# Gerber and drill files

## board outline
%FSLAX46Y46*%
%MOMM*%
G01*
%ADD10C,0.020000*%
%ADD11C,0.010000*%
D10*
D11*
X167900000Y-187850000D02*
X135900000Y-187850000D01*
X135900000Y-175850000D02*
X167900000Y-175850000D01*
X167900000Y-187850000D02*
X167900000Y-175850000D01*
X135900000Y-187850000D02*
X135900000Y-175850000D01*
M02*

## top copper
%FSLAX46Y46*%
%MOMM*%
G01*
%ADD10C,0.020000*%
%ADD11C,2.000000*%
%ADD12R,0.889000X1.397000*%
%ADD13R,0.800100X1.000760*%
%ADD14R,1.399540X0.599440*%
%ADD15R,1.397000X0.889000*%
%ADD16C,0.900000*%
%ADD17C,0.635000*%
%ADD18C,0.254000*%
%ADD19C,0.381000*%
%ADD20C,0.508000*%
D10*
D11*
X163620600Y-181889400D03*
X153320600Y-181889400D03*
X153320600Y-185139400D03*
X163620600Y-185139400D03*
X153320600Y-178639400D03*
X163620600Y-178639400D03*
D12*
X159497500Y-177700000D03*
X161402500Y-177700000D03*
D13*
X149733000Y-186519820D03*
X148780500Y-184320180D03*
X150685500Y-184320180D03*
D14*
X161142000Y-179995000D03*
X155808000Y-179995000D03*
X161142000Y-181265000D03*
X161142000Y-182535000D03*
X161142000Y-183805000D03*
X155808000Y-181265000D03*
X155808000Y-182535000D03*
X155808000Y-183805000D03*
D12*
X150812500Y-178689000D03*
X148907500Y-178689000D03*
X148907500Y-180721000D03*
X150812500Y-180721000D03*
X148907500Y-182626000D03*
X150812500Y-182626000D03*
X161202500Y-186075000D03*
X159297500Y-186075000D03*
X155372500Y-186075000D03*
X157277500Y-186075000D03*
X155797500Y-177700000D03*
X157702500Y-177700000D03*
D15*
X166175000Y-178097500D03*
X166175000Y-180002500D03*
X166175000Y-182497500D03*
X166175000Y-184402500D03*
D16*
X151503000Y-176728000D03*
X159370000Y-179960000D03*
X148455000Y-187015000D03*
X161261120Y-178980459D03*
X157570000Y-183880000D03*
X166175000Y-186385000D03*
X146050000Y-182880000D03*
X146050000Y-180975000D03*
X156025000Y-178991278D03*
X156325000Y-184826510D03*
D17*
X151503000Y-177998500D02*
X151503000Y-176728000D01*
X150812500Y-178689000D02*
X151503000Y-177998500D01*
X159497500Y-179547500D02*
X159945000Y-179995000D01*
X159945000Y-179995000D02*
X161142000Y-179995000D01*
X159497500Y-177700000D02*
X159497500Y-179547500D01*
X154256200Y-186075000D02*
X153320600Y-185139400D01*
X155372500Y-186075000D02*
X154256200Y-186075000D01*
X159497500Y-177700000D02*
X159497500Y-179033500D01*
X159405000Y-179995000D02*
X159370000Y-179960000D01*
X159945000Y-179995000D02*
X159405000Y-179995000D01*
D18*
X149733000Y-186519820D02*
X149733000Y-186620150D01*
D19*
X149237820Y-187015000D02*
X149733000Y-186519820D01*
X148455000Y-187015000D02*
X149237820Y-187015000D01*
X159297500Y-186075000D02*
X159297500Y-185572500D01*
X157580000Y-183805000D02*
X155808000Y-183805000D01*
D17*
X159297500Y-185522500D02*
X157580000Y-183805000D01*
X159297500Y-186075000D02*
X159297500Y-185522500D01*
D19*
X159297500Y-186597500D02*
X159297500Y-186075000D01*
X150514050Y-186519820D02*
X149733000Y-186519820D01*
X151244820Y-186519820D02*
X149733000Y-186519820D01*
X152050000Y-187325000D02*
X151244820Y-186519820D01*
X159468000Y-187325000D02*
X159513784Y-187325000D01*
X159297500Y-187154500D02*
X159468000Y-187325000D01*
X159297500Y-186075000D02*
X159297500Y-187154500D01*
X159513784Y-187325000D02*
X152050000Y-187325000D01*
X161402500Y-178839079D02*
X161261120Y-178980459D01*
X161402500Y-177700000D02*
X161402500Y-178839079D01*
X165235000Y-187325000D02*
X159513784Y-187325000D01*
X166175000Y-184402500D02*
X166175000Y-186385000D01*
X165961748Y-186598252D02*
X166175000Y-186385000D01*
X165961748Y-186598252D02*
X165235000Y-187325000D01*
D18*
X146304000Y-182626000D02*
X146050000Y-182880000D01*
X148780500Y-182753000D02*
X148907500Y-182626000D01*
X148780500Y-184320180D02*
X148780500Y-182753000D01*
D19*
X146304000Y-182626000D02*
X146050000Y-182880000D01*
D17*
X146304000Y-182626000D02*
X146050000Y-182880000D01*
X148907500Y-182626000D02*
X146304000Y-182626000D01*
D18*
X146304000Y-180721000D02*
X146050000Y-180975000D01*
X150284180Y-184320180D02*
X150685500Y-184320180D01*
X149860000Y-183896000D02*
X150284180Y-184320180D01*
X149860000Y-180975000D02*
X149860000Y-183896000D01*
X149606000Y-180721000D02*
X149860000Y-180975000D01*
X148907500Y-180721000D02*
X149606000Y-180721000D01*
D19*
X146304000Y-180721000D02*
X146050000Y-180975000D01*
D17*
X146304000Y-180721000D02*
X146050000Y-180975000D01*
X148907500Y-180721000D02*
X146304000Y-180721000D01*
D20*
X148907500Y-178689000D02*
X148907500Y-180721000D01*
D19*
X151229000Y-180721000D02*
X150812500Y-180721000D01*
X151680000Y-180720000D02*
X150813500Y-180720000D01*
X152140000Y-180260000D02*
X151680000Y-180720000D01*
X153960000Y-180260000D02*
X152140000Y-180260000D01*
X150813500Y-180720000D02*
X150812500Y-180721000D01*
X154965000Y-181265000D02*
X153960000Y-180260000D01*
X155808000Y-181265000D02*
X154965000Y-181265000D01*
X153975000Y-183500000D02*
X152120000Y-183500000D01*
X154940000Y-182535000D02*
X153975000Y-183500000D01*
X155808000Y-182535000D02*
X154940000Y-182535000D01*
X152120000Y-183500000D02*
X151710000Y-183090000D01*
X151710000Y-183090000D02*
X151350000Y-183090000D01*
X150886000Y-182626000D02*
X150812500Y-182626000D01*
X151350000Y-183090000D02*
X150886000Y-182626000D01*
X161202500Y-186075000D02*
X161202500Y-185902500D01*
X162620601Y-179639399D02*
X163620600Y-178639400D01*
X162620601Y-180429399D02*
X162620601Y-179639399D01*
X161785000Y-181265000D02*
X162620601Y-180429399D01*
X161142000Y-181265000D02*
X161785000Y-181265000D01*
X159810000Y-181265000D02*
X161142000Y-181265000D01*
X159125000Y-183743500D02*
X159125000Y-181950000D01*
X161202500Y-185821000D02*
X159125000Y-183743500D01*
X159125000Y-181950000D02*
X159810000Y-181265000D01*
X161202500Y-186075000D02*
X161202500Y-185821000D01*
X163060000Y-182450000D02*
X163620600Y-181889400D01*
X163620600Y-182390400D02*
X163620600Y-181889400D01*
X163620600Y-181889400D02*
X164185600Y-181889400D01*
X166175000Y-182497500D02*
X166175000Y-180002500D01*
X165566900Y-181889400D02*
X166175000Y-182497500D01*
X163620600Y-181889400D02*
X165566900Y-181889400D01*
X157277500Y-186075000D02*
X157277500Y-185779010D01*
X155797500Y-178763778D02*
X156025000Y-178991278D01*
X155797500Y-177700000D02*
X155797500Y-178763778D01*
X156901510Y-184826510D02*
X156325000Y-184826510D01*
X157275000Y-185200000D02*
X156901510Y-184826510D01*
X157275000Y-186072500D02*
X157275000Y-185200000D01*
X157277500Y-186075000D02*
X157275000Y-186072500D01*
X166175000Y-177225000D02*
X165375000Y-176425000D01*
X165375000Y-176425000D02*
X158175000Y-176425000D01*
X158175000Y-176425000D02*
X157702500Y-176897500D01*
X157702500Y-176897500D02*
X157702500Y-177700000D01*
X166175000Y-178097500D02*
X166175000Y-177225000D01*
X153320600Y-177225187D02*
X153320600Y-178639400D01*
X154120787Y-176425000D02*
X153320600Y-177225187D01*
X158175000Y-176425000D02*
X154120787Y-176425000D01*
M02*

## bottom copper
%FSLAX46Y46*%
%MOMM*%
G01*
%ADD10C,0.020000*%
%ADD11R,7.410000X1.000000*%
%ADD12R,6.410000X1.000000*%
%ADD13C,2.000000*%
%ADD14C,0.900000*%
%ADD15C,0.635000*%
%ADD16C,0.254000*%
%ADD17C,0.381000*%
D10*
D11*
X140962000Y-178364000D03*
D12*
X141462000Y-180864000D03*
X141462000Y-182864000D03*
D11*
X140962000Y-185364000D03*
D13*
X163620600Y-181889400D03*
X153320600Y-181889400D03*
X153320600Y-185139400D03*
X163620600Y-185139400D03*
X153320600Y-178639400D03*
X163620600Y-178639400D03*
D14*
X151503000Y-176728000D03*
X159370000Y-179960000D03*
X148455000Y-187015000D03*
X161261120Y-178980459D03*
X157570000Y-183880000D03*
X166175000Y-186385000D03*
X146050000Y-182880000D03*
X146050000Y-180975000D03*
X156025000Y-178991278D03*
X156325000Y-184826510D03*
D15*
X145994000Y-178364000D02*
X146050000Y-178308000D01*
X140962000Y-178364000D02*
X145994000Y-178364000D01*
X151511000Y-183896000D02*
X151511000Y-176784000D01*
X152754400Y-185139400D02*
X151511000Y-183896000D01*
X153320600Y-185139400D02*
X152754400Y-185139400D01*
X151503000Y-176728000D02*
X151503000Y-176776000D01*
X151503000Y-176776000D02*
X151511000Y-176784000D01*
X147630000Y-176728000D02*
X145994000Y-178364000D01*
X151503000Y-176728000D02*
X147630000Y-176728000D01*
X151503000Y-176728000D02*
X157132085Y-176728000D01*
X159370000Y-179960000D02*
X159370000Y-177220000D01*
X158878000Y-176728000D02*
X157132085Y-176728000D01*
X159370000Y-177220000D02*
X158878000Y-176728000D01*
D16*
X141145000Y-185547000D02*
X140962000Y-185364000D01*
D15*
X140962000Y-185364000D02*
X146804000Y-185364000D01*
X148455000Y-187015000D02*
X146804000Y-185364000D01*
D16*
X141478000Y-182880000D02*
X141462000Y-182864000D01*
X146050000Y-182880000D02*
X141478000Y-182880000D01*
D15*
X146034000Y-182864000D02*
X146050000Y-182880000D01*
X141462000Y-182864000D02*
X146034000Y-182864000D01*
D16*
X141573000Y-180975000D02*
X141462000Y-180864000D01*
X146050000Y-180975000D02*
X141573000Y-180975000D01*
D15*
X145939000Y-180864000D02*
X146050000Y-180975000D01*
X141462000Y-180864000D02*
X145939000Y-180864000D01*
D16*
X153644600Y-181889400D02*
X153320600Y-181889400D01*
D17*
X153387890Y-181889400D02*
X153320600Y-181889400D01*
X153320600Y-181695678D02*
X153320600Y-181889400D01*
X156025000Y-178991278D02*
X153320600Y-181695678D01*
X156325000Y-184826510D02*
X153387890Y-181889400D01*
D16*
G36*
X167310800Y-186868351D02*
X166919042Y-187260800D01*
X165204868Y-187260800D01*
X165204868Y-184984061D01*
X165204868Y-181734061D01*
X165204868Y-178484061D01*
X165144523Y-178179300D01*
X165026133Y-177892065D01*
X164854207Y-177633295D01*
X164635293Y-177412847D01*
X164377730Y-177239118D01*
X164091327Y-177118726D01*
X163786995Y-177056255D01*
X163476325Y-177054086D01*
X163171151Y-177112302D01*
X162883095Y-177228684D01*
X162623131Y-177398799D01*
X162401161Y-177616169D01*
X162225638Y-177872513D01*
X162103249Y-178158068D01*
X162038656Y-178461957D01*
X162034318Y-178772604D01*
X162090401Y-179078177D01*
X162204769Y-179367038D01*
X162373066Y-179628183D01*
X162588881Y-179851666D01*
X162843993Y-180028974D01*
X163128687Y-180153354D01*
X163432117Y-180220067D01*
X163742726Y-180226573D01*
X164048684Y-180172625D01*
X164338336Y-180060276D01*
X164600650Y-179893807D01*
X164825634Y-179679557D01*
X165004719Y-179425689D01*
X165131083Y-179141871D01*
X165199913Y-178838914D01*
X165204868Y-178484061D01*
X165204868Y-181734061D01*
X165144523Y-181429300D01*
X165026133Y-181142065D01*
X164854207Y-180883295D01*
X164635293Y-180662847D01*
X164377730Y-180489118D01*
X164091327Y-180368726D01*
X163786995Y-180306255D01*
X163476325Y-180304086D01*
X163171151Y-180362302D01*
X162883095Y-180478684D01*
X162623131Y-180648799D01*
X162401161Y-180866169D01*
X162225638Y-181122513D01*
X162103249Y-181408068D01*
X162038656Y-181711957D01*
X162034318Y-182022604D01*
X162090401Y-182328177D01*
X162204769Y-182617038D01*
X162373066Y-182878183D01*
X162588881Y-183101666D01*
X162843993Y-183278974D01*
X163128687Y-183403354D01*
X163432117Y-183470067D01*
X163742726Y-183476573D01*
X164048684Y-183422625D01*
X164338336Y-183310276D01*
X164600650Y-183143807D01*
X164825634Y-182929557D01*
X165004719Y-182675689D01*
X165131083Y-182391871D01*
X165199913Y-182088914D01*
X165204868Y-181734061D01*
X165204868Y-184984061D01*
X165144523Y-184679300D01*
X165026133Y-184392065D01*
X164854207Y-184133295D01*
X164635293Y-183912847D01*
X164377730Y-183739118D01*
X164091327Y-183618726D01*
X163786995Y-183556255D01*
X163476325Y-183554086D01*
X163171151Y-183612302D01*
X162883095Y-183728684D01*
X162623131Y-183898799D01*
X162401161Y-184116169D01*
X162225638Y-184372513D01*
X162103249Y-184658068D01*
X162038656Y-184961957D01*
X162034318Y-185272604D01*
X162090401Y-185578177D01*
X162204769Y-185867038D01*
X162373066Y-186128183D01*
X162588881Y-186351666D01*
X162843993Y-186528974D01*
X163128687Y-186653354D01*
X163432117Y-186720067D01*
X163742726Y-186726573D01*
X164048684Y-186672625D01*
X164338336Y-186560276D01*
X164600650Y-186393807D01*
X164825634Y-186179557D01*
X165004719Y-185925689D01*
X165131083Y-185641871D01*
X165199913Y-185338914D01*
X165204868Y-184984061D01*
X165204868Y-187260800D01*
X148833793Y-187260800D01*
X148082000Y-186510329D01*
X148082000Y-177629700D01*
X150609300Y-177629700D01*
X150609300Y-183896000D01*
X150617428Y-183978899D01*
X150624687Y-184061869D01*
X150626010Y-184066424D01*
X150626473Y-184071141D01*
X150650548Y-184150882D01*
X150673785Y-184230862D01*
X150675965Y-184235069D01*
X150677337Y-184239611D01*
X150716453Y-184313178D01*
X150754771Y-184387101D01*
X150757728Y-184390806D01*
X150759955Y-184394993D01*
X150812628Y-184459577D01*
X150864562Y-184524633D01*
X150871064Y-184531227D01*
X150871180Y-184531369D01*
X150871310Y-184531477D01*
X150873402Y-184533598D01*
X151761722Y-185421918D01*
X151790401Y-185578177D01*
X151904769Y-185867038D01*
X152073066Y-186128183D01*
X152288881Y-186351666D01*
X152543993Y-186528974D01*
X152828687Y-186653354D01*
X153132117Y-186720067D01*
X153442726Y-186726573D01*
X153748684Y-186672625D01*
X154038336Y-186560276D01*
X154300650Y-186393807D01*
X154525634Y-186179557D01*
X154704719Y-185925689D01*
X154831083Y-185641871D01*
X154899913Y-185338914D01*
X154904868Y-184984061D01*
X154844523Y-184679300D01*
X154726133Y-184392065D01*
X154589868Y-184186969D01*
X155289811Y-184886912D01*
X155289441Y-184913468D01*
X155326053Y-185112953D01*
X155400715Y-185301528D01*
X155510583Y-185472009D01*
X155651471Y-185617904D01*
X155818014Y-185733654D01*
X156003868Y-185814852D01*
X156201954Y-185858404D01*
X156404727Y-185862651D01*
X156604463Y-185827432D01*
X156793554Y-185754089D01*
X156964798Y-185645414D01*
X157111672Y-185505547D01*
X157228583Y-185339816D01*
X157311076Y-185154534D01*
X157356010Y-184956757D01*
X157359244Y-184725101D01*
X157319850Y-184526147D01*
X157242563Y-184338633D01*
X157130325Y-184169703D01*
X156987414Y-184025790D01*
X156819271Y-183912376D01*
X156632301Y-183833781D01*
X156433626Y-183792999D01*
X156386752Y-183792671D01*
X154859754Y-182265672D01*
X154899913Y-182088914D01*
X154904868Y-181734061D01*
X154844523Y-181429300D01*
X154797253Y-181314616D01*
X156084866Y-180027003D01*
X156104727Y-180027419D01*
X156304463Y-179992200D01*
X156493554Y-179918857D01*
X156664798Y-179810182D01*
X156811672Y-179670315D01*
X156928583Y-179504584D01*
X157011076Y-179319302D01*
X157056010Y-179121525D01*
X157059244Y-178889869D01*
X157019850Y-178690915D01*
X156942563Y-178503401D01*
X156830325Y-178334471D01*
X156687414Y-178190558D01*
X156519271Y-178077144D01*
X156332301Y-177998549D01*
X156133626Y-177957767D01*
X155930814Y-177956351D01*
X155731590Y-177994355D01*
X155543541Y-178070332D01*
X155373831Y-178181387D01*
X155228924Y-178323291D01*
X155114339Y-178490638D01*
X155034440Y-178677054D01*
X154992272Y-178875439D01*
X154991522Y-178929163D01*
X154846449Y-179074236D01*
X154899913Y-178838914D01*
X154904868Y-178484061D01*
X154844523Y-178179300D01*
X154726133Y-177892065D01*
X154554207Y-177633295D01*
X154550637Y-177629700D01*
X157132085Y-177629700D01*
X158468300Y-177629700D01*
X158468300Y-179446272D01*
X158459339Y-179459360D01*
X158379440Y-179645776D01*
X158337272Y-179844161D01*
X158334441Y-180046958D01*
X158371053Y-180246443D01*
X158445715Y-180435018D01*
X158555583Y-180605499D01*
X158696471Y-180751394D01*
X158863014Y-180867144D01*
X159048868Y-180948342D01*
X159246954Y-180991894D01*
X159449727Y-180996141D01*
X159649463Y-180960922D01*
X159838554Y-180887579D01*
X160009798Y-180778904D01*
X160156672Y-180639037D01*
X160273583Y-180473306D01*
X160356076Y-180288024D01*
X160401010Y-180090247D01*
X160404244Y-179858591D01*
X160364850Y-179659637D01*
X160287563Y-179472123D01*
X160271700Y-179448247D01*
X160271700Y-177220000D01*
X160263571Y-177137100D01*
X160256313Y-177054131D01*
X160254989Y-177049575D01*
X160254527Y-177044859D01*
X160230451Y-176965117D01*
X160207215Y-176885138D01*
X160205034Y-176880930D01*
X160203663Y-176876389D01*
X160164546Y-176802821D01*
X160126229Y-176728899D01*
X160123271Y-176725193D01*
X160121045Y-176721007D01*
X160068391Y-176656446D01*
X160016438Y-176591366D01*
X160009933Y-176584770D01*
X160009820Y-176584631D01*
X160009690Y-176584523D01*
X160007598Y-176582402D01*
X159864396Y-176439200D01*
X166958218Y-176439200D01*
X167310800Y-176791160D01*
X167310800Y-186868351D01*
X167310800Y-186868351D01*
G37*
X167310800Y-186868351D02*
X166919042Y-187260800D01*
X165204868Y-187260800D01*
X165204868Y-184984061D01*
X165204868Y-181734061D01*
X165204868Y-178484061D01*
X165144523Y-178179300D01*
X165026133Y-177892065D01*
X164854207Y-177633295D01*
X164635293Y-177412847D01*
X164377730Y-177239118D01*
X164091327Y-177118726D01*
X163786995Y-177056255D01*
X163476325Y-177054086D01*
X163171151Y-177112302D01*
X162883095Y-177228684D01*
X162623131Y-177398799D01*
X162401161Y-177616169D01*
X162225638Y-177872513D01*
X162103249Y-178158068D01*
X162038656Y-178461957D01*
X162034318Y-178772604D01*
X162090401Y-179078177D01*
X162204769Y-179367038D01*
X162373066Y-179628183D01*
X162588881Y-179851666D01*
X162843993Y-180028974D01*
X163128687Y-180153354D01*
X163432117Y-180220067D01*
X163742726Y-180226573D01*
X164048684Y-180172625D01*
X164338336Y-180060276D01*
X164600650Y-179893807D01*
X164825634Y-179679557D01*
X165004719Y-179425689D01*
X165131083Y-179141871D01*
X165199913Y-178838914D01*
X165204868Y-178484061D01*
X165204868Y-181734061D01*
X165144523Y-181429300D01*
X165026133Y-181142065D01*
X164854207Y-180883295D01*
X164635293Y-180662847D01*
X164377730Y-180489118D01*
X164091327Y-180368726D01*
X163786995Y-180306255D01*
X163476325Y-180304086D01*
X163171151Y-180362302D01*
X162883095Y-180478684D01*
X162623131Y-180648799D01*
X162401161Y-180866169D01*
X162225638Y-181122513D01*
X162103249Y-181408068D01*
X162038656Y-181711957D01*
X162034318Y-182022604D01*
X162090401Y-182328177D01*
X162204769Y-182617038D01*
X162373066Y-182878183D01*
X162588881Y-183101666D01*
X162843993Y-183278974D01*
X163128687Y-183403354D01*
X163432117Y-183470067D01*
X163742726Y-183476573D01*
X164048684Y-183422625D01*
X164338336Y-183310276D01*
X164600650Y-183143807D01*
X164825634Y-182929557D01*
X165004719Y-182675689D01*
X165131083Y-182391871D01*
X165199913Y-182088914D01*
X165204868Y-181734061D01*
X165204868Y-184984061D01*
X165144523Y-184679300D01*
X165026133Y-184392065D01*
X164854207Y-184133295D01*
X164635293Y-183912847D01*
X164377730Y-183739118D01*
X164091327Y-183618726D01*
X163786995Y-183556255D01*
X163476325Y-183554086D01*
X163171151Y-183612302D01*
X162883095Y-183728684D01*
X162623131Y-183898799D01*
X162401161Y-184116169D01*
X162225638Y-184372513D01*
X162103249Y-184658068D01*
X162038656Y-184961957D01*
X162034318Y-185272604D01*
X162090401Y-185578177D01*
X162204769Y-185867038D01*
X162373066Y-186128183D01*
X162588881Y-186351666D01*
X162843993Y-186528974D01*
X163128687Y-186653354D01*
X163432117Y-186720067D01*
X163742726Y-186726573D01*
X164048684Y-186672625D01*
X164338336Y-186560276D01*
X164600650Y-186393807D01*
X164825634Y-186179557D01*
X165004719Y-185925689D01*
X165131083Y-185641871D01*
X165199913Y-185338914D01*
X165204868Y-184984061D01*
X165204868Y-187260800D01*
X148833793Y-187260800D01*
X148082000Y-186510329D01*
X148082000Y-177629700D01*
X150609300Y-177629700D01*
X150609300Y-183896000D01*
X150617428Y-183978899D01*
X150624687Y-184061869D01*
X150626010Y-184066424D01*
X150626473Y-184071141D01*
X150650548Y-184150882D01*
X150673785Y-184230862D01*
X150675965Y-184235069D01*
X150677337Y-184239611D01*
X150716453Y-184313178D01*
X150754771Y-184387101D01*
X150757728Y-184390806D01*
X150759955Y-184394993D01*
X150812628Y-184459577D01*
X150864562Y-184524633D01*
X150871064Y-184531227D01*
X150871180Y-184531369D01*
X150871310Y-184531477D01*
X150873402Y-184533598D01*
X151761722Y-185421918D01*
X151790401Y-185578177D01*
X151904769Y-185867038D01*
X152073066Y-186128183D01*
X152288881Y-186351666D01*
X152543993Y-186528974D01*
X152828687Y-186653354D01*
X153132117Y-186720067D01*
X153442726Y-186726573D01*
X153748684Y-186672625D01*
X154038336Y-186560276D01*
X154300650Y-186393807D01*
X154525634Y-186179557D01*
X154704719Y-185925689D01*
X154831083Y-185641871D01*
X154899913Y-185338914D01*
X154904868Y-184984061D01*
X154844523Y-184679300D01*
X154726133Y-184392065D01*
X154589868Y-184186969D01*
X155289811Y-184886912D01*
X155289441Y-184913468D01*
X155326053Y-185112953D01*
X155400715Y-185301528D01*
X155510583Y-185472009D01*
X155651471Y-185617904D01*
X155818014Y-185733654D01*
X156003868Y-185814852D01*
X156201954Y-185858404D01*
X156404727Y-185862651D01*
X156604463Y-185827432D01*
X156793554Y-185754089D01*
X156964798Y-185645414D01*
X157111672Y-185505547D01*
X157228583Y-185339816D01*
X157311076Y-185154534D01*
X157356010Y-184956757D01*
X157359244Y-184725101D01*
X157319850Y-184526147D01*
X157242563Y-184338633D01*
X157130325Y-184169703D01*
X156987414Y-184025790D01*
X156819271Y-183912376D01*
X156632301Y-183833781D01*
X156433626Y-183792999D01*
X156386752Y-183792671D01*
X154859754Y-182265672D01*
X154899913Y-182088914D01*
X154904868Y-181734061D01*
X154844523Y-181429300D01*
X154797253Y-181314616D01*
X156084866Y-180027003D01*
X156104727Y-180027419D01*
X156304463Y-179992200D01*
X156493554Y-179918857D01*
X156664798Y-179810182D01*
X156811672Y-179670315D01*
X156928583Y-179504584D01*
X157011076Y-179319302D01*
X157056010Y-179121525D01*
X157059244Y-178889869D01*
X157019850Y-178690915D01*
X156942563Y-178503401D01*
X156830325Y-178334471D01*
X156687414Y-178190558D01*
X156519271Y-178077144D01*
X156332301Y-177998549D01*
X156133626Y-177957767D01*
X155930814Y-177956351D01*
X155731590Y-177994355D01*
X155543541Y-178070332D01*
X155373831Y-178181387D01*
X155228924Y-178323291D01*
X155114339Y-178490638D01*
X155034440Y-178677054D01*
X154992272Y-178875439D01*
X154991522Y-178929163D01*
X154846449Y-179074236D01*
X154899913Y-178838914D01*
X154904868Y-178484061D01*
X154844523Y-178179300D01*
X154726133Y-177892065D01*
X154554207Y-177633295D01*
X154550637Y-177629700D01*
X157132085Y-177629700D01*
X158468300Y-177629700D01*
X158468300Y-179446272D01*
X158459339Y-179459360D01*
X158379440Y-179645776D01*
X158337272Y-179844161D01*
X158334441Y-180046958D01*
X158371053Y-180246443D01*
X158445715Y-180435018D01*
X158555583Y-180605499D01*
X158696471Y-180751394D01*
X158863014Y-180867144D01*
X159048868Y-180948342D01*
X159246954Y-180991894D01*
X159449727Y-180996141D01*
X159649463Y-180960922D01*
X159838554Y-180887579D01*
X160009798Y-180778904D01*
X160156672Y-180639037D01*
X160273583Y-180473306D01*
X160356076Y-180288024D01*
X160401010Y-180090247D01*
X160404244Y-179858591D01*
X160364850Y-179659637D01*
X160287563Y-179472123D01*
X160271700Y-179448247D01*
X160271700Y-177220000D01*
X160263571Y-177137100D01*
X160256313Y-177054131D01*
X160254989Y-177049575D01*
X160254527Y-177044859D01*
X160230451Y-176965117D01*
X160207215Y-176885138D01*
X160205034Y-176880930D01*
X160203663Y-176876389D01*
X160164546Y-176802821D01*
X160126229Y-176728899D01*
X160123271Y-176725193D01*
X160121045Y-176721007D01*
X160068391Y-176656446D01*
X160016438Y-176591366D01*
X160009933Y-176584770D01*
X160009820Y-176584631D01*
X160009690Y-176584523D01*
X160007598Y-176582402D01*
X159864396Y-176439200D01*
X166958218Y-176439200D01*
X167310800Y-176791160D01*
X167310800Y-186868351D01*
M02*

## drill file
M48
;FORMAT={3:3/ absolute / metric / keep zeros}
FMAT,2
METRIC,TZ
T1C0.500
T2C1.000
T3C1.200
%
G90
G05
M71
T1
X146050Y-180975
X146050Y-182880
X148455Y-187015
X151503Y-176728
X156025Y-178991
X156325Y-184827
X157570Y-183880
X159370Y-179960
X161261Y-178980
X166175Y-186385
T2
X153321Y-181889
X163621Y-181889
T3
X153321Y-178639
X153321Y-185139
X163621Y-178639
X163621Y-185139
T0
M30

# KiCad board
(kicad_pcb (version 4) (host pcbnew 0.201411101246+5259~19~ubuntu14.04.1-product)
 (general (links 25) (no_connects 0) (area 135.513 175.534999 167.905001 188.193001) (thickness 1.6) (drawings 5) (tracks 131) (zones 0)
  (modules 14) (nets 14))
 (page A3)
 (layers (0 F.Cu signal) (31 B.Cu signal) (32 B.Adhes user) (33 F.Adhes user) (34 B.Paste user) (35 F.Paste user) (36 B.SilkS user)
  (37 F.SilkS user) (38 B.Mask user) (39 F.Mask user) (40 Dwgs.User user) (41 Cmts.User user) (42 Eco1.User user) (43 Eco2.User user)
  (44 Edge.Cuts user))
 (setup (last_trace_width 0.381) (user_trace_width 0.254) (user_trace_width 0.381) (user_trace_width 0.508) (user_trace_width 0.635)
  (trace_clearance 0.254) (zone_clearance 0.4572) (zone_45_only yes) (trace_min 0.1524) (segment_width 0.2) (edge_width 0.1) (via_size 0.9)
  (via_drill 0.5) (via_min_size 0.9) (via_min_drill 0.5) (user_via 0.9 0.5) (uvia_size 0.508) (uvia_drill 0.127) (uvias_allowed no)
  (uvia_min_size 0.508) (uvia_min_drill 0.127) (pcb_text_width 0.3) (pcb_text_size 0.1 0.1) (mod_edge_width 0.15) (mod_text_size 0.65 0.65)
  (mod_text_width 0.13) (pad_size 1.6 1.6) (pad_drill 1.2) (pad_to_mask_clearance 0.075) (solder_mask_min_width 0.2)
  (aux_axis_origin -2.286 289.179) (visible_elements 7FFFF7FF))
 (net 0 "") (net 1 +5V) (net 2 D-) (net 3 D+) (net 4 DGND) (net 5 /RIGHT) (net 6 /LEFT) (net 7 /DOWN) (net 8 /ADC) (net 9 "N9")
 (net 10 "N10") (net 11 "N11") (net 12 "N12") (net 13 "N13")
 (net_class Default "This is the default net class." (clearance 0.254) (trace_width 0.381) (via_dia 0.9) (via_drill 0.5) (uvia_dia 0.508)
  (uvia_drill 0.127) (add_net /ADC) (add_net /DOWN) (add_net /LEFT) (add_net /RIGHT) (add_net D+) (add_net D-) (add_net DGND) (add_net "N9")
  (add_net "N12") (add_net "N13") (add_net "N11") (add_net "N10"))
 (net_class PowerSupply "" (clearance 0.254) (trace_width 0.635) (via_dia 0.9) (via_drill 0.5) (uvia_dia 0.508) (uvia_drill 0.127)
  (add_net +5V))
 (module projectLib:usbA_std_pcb (layer B.Cu) (at 136.017 181.864)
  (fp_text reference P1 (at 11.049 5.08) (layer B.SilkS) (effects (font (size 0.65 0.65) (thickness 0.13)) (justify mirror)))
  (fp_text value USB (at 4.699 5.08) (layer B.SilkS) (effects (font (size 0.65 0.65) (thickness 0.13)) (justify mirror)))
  (pad 1 smd rect (at 4.945 -3.5) (size 7.41 1) (layers B.Cu B.Mask) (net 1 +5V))
  (pad 2 smd rect (at 5.445 -1) (size 6.41 1) (layers B.Cu B.Mask) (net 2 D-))
  (pad 3 smd rect (at 5.445 1) (size 6.41 1) (layers B.Cu B.Mask) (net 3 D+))
  (pad 4 smd rect (at 4.945 3.5) (size 7.41 1) (layers B.Cu B.Mask) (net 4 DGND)))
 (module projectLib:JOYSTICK (layer B.Cu) (at 158.4706 181.8894)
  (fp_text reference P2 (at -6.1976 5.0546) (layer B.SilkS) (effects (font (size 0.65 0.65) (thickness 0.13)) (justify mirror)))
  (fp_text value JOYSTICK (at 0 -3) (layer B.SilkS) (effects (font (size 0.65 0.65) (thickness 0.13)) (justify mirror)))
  (pad 5 thru_hole circle (at 5.15 0) (size 2 2) (drill 1) (layers *.Cu *.Mask B.SilkS) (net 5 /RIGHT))
  (pad 2 thru_hole circle (at -5.15 0) (size 2 2) (drill 1) (layers *.Cu *.Mask B.SilkS) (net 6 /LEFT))
  (pad 1 thru_hole circle (at -5.15 3.25) (size 2 2) (drill 1.2) (layers *.Cu *.Mask B.SilkS) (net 1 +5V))
  (pad 6 thru_hole circle (at 5.15 3.25) (size 2 2) (drill 1.2) (layers *.Cu *.Mask B.SilkS))
  (pad 3 thru_hole circle (at -5.15 -3.25) (size 2 2) (drill 1.2) (layers *.Cu *.Mask B.SilkS) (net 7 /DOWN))
  (pad 4 thru_hole circle (at 5.15 -3.25) (size 2 2) (drill 1.2) (layers *.Cu *.Mask B.SilkS) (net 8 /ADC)))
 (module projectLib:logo (layer F.Cu) (at 140.7 181.66 90)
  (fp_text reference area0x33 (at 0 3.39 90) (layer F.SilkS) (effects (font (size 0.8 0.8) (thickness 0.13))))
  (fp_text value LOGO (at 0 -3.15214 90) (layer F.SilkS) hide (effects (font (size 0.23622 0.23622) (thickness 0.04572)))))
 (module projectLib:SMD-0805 (layer F.Cu) (at 160.45 177.7)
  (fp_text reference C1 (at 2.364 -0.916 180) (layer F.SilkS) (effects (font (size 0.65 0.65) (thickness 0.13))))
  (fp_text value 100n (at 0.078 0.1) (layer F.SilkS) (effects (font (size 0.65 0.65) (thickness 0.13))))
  (pad 1 smd rect (at -0.9525 0) (size 0.889 1.397) (layers F.Cu F.Paste F.Mask) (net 1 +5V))
  (pad 2 smd rect (at 0.9525 0) (size 0.889 1.397) (layers F.Cu F.Paste F.Mask) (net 4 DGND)))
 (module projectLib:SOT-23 (layer F.Cu) (at 149.733 185.42 180)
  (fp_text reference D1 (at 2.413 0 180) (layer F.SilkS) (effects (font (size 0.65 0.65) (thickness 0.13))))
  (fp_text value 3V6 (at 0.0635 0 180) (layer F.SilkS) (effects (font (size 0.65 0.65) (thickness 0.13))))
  (pad 3 smd rect (at 0 -1.09982 180) (size 0.8001 1.00076) (layers F.Cu F.Paste F.Mask) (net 4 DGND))
  (pad 2 smd rect (at 0.9525 1.09982 180) (size 0.8001 1.00076) (layers F.Cu F.Paste F.Mask) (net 3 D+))
  (pad 1 smd rect (at -0.9525 1.09982 180) (size 0.8001 1.00076) (layers F.Cu F.Paste F.Mask) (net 2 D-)))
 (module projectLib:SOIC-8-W (layer F.Cu) (at 158.475 181.9 270)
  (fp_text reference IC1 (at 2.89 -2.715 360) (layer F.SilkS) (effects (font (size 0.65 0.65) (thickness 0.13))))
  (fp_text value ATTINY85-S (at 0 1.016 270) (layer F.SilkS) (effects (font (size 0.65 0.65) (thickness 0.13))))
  (pad 8 smd rect (at -1.905 -2.667 270) (size 0.59944 1.39954) (layers F.Cu F.Paste F.Mask) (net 1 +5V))
  (pad 1 smd rect (at -1.905 2.667 270) (size 0.59944 1.39954) (layers F.Cu F.Paste F.Mask) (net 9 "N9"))
  (pad 7 smd rect (at -0.635 -2.667 270) (size 0.59944 1.39954) (layers F.Cu F.Paste F.Mask) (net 8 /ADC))
  (pad 6 smd rect (at 0.635 -2.667 270) (size 0.59944 1.39954) (layers F.Cu F.Paste F.Mask) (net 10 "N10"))
  (pad 5 smd rect (at 1.905 -2.667 270) (size 0.59944 1.39954) (layers F.Cu F.Paste F.Mask) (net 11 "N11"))
  (pad 2 smd rect (at -0.635 2.667 270) (size 0.59944 1.39954) (layers F.Cu F.Paste F.Mask) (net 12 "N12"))
  (pad 3 smd rect (at 0.635 2.667 270) (size 0.59944 1.39954) (layers F.Cu F.Paste F.Mask) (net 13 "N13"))
  (pad 4 smd rect (at 1.905 2.667 270) (size 0.59944 1.39954) (layers F.Cu F.Paste F.Mask) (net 4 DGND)))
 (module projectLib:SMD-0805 (layer F.Cu) (at 149.86 178.689 180)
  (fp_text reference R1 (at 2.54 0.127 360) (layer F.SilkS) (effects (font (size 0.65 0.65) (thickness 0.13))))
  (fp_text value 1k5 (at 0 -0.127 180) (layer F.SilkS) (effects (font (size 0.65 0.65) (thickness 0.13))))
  (pad 1 smd rect (at -0.9525 0 180) (size 0.889 1.397) (layers F.Cu F.Paste F.Mask) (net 1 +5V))
  (pad 2 smd rect (at 0.9525 0 180) (size 0.889 1.397) (layers F.Cu F.Paste F.Mask) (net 2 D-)))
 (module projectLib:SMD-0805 (layer F.Cu) (at 149.86 180.721)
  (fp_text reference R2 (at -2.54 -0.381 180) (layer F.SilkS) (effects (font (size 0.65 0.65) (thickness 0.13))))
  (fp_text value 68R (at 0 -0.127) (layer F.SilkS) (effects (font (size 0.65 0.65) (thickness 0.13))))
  (pad 1 smd rect (at -0.9525 0) (size 0.889 1.397) (layers F.Cu F.Paste F.Mask) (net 2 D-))
  (pad 2 smd rect (at 0.9525 0) (size 0.889 1.397) (layers F.Cu F.Paste F.Mask) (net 12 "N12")))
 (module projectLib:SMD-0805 (layer F.Cu) (at 149.86 182.626)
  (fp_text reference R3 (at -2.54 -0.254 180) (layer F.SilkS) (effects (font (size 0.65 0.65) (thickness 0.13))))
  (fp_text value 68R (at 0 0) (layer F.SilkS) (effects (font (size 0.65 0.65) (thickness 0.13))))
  (pad 1 smd rect (at -0.9525 0) (size 0.889 1.397) (layers F.Cu F.Paste F.Mask) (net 3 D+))
  (pad 2 smd rect (at 0.9525 0) (size 0.889 1.397) (layers F.Cu F.Paste F.Mask) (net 13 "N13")))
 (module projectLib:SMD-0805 (layer F.Cu) (at 160.25 186.075 180)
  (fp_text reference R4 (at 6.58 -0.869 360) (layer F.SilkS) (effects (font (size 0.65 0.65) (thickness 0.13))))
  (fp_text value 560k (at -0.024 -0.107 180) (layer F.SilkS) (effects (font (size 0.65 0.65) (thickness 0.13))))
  (pad 1 smd rect (at -0.9525 0 180) (size 0.889 1.397) (layers F.Cu F.Paste F.Mask) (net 8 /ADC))
  (pad 2 smd rect (at 0.9525 0 180) (size 0.889 1.397) (layers F.Cu F.Paste F.Mask) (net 4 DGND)))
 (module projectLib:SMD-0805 (layer F.Cu) (at 156.325 186.075)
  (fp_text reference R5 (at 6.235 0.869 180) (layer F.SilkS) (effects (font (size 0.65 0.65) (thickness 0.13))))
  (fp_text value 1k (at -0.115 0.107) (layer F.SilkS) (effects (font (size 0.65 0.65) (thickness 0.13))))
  (pad 1 smd rect (at -0.9525 0) (size 0.889 1.397) (layers F.Cu F.Paste F.Mask) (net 1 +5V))
  (pad 2 smd rect (at 0.9525 0) (size 0.889 1.397) (layers F.Cu F.Paste F.Mask) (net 6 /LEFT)))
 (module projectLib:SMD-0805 (layer F.Cu) (at 156.75 177.7)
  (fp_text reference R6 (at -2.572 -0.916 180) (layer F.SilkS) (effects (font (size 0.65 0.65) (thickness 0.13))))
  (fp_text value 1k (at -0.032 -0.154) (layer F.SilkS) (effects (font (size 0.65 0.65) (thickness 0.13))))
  (pad 1 smd rect (at -0.9525 0) (size 0.889 1.397) (layers F.Cu F.Paste F.Mask) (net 6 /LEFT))
  (pad 2 smd rect (at 0.9525 0) (size 0.889 1.397) (layers F.Cu F.Paste F.Mask) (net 7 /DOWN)))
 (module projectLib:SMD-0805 (layer F.Cu) (at 166.175 179.05 270)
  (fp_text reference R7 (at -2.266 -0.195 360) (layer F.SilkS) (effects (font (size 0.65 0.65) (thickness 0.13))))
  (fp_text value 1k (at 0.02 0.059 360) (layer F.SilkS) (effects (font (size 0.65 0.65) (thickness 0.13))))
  (pad 1 smd rect (at -0.9525 0 270) (size 0.889 1.397) (layers F.Cu F.Paste F.Mask) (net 7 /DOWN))
  (pad 2 smd rect (at 0.9525 0 270) (size 0.889 1.397) (layers F.Cu F.Paste F.Mask) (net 5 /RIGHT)))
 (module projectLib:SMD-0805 (layer F.Cu) (at 166.175 183.45 270)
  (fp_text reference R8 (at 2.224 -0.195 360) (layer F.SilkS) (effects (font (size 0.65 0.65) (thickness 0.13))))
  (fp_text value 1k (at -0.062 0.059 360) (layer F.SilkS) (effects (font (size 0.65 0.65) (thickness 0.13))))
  (pad 1 smd rect (at -0.9525 0 270) (size 0.889 1.397) (layers F.Cu F.Paste F.Mask) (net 5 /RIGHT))
  (pad 2 smd rect (at 0.9525 0 270) (size 0.889 1.397) (layers F.Cu F.Paste F.Mask) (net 4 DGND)))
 (gr_line (start 167.9 187.85) (end 135.9 187.85) (angle 90) (layer Edge.Cuts) (width 0.01))
 (gr_line (start 135.9 175.85) (end 167.9 175.85) (angle 90) (layer Edge.Cuts) (width 0.01))
 (gr_line (start 167.9 187.85) (end 167.9 175.85) (angle 90) (layer Edge.Cuts) (width 0.01))
 (gr_line (start 135.9 187.85) (end 135.9 175.85) (angle 90) (layer Edge.Cuts) (width 0.01))
 (segment (start 159.37 177.22) (end 158.878 176.728) (width 0.635) (layer B.Cu) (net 1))
 (segment (start 158.878 176.728) (end 157.132085 176.728) (width 0.635) (layer B.Cu) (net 1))
 (segment (start 159.37 179.96) (end 159.37 177.22) (width 0.635) (layer B.Cu) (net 1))
 (segment (start 159.945 179.995) (end 159.405 179.995) (width 0.635) (layer F.Cu) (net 1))
 (segment (start 159.405 179.995) (end 159.37 179.96) (width 0.635) (layer F.Cu) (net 1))
 (via (at 159.37 179.96) (size 0.9) (drill 0.5) (layers F.Cu B.Cu) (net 1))
 (segment (start 151.503 176.728) (end 157.132085 176.728) (width 0.635) (layer B.Cu) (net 1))
 (segment (start 159.4975 177.7) (end 159.4975 179.0335) (width 0.635) (layer F.Cu) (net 1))
 (segment (start 155.3725 186.075) (end 154.2562 186.075) (width 0.635) (layer F.Cu) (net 1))
 (segment (start 154.2562 186.075) (end 153.3206 185.1394) (width 0.635) (layer F.Cu) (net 1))
 (segment (start 159.4975 177.7) (end 159.4975 179.5475) (width 0.635) (layer F.Cu) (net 1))
 (segment (start 159.945 179.995) (end 161.142 179.995) (width 0.635) (layer F.Cu) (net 1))
 (segment (start 159.4975 179.5475) (end 159.945 179.995) (width 0.635) (layer F.Cu) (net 1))
 (segment (start 151.503 176.728) (end 147.63 176.728) (width 0.635) (layer B.Cu) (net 1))
 (segment (start 147.63 176.728) (end 145.994 178.364) (width 0.635) (layer B.Cu) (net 1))
 (segment (start 150.8125 178.689) (end 151.503 177.9985) (width 0.635) (layer F.Cu) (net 1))
 (segment (start 151.503 176.776) (end 151.511 176.784) (width 0.635) (layer B.Cu) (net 1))
 (segment (start 151.503 176.728) (end 151.503 176.776) (width 0.635) (layer B.Cu) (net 1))
 (via (at 151.503 176.728) (size 0.9) (drill 0.5) (layers F.Cu B.Cu) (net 1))
 (segment (start 151.503 177.9985) (end 151.503 176.728) (width 0.635) (layer F.Cu) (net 1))
 (segment (start 153.3206 185.1394) (end 152.7544 185.1394) (width 0.635) (layer B.Cu) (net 1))
 (segment (start 152.7544 185.1394) (end 151.511 183.896) (width 0.635) (layer B.Cu) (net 1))
 (segment (start 151.511 183.896) (end 151.511 176.784) (width 0.635) (layer B.Cu) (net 1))
 (segment (start 140.962 178.364) (end 145.994 178.364) (width 0.635) (layer B.Cu) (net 1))
 (segment (start 145.994 178.364) (end 146.05 178.308) (width 0.635) (layer B.Cu) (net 1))
 (segment (start 165.961748 186.598252) (end 165.235 187.325) (width 0.381) (layer F.Cu) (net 4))
 (segment (start 165.961748 186.598252) (end 166.175 186.385) (width 0.381) (layer F.Cu) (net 4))
 (via (at 166.175 186.385) (size 0.9) (drill 0.5) (layers F.Cu B.Cu) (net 4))
 (segment (start 166.175 184.4025) (end 166.175 186.385) (width 0.381) (layer F.Cu) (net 4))
 (segment (start 165.235 187.325) (end 159.513784 187.325) (width 0.381) (layer F.Cu) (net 4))
 (via (at 157.57 183.88) (size 0.9) (drill 0.5) (layers F.Cu B.Cu) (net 4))
 (segment (start 161.4025 177.7) (end 161.4025 178.839079) (width 0.381) (layer F.Cu) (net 4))
 (segment (start 161.4025 178.839079) (end 161.26112 178.980459) (width 0.381) (layer F.Cu) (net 4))
 (via (at 161.26112 178.980459) (size 0.9) (drill 0.5) (layers F.Cu B.Cu) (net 4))
 (segment (start 159.513784 187.325) (end 152.05 187.325) (width 0.381) (layer F.Cu) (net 4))
 (segment (start 159.2975 186.075) (end 159.2975 187.1545) (width 0.381) (layer F.Cu) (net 4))
 (segment (start 159.2975 187.1545) (end 159.468 187.325) (width 0.381) (layer F.Cu) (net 4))
 (segment (start 159.468 187.325) (end 159.513784 187.325) (width 0.381) (layer F.Cu) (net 4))
 (segment (start 152.05 187.325) (end 151.24482 186.51982) (width 0.381) (layer F.Cu) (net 4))
 (segment (start 151.24482 186.51982) (end 149.733 186.51982) (width 0.381) (layer F.Cu) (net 4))
 (segment (start 150.51405 186.51982) (end 149.733 186.51982) (width 0.381) (layer F.Cu) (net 4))
 (segment (start 159.2975 186.5975) (end 159.2975 186.075) (width 0.381) (layer F.Cu) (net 4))
 (segment (start 159.2975 186.075) (end 159.2975 185.5225) (width 0.635) (layer F.Cu) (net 4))
 (segment (start 159.2975 185.5225) (end 157.58 183.805) (width 0.635) (layer F.Cu) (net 4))
 (segment (start 157.58 183.805) (end 155.808 183.805) (width 0.381) (layer F.Cu) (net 4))
 (segment (start 159.2975 186.075) (end 159.2975 185.5725) (width 0.381) (layer F.Cu) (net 4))
 (segment (start 148.455 187.015) (end 146.804 185.364) (width 0.635) (layer B.Cu) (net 4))
 (segment (start 148.455 187.015) (end 149.23782 187.015) (width 0.381) (layer F.Cu) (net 4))
 (segment (start 149.23782 187.015) (end 149.733 186.51982) (width 0.381) (layer F.Cu) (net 4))
 (segment (start 140.962 185.364) (end 146.804 185.364) (width 0.635) (layer B.Cu) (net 4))
 (via (at 148.455 187.015) (size 0.9) (drill 0.5) (layers F.Cu B.Cu) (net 4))
 (segment (start 141.145 185.547) (end 140.962 185.364) (width 0.254) (layer B.Cu) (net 4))
 (segment (start 149.733 186.51982) (end 149.733 186.62015) (width 0.254) (layer F.Cu) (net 4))
 (segment (start 148.9075 182.626) (end 146.304 182.626) (width 0.635) (layer F.Cu) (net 3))
 (segment (start 146.304 182.626) (end 146.05 182.88) (width 0.635) (layer F.Cu) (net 3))
 (segment (start 141.462 182.864) (end 146.034 182.864) (width 0.635) (layer B.Cu) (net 3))
 (segment (start 146.034 182.864) (end 146.05 182.88) (width 0.635) (layer B.Cu) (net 3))
 (segment (start 146.304 182.626) (end 146.05 182.88) (width 0.381) (layer F.Cu) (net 3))
 (segment (start 148.7805 184.32018) (end 148.7805 182.753) (width 0.254) (layer F.Cu) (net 3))
 (segment (start 148.7805 182.753) (end 148.9075 182.626) (width 0.254) (layer F.Cu) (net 3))
 (segment (start 146.05 182.88) (end 141.478 182.88) (width 0.254) (layer B.Cu) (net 3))
 (segment (start 141.478 182.88) (end 141.462 182.864) (width 0.254) (layer B.Cu) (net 3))
 (segment (start 146.304 182.626) (end 146.05 182.88) (width 0.254) (layer F.Cu) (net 3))
 (via (at 146.05 182.88) (size 0.9) (drill 0.5) (layers F.Cu B.Cu) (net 3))
 (segment (start 148.9075 178.689) (end 148.9075 180.721) (width 0.508) (layer F.Cu) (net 2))
 (segment (start 148.9075 180.721) (end 146.304 180.721) (width 0.635) (layer F.Cu) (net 2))
 (segment (start 146.304 180.721) (end 146.05 180.975) (width 0.635) (layer F.Cu) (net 2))
 (segment (start 141.462 180.864) (end 145.939 180.864) (width 0.635) (layer B.Cu) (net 2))
 (segment (start 145.939 180.864) (end 146.05 180.975) (width 0.635) (layer B.Cu) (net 2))
 (segment (start 146.304 180.721) (end 146.05 180.975) (width 0.381) (layer F.Cu) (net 2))
 (segment (start 148.9075 180.721) (end 149.606 180.721) (width 0.254) (layer F.Cu) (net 2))
 (segment (start 149.606 180.721) (end 149.86 180.975) (width 0.254) (layer F.Cu) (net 2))
 (segment (start 149.86 180.975) (end 149.86 183.896) (width 0.254) (layer F.Cu) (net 2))
 (segment (start 149.86 183.896) (end 150.28418 184.32018) (width 0.254) (layer F.Cu) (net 2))
 (segment (start 150.28418 184.32018) (end 150.6855 184.32018) (width 0.254) (layer F.Cu) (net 2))
 (segment (start 146.05 180.975) (end 141.573 180.975) (width 0.254) (layer B.Cu) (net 2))
 (via (at 146.05 180.975) (size 0.9) (drill 0.5) (layers F.Cu B.Cu) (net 2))
 (segment (start 146.304 180.721) (end 146.05 180.975) (width 0.254) (layer F.Cu) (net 2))
 (segment (start 141.573 180.975) (end 141.462 180.864) (width 0.254) (layer B.Cu) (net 2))
 (segment (start 155.808 181.265) (end 154.965 181.265) (width 0.381) (layer F.Cu) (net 12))
 (segment (start 154.965 181.265) (end 153.96 180.26) (width 0.381) (layer F.Cu) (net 12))
 (segment (start 150.8135 180.72) (end 150.8125 180.721) (width 0.381) (layer F.Cu) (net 12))
 (segment (start 153.96 180.26) (end 152.14 180.26) (width 0.381) (layer F.Cu) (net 12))
 (segment (start 152.14 180.26) (end 151.68 180.72) (width 0.381) (layer F.Cu) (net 12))
 (segment (start 151.68 180.72) (end 150.8135 180.72) (width 0.381) (layer F.Cu) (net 12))
 (segment (start 151.229 180.721) (end 150.8125 180.721) (width 0.381) (layer F.Cu) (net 12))
 (segment (start 151.35 183.09) (end 150.886 182.626) (width 0.381) (layer F.Cu) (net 13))
 (segment (start 150.886 182.626) (end 150.8125 182.626) (width 0.381) (layer F.Cu) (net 13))
 (segment (start 151.71 183.09) (end 151.35 183.09) (width 0.381) (layer F.Cu) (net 13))
 (segment (start 152.12 183.5) (end 151.71 183.09) (width 0.381) (layer F.Cu) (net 13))
 (segment (start 155.808 182.535) (end 154.94 182.535) (width 0.381) (layer F.Cu) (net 13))
 (segment (start 154.94 182.535) (end 153.975 183.5) (width 0.381) (layer F.Cu) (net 13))
 (segment (start 153.975 183.5) (end 152.12 183.5) (width 0.381) (layer F.Cu) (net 13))
 (segment (start 161.2025 186.075) (end 161.2025 185.821) (width 0.381) (layer F.Cu) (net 8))
 (segment (start 159.125 181.95) (end 159.81 181.265) (width 0.381) (layer F.Cu) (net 8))
 (segment (start 161.2025 185.821) (end 159.125 183.7435) (width 0.381) (layer F.Cu) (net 8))
 (segment (start 159.125 183.7435) (end 159.125 181.95) (width 0.381) (layer F.Cu) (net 8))
 (segment (start 159.81 181.265) (end 161.142 181.265) (width 0.381) (layer F.Cu) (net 8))
 (segment (start 161.142 181.265) (end 161.785 181.265) (width 0.381) (layer F.Cu) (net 8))
 (segment (start 161.785 181.265) (end 162.620601 180.429399) (width 0.381) (layer F.Cu) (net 8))
 (segment (start 162.620601 180.429399) (end 162.620601 179.639399) (width 0.381) (layer F.Cu) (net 8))
 (segment (start 162.620601 179.639399) (end 163.6206 178.6394) (width 0.381) (layer F.Cu) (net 8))
 (segment (start 161.2025 186.075) (end 161.2025 185.9025) (width 0.381) (layer F.Cu) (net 8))
 (segment (start 163.6206 181.8894) (end 165.5669 181.8894) (width 0.381) (layer F.Cu) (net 5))
 (segment (start 165.5669 181.8894) (end 166.175 182.4975) (width 0.381) (layer F.Cu) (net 5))
 (segment (start 166.175 182.4975) (end 166.175 180.0025) (width 0.381) (layer F.Cu) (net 5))
 (segment (start 163.6206 181.8894) (end 164.1856 181.8894) (width 0.381) (layer F.Cu) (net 5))
 (segment (start 163.6206 182.3904) (end 163.6206 181.8894) (width 0.381) (layer F.Cu) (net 5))
 (segment (start 163.06 182.45) (end 163.6206 181.8894) (width 0.381) (layer F.Cu) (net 5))
 (segment (start 157.2775 186.075) (end 157.275 186.0725) (width 0.381) (layer F.Cu) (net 6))
 (segment (start 157.275 186.0725) (end 157.275 185.2) (width 0.381) (layer F.Cu) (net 6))
 (segment (start 157.275 185.2) (end 156.90151 184.82651) (width 0.381) (layer F.Cu) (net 6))
 (segment (start 156.90151 184.82651) (end 156.325 184.82651) (width 0.381) (layer F.Cu) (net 6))
 (via (at 156.325 184.82651) (size 0.9) (drill 0.5) (layers F.Cu B.Cu) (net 6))
 (segment (start 156.325 184.82651) (end 153.38789 181.8894) (width 0.381) (layer B.Cu) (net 6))
 (segment (start 156.025 178.991278) (end 153.3206 181.695678) (width 0.381) (layer B.Cu) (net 6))
 (segment (start 153.3206 181.695678) (end 153.3206 181.8894) (width 0.381) (layer B.Cu) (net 6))
 (segment (start 155.7975 177.7) (end 155.7975 178.763778) (width 0.381) (layer F.Cu) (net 6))
 (segment (start 155.7975 178.763778) (end 156.025 178.991278) (width 0.381) (layer F.Cu) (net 6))
 (via (at 156.025 178.991278) (size 0.9) (drill 0.5) (layers F.Cu B.Cu) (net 6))
 (segment (start 153.38789 181.8894) (end 153.3206 181.8894) (width 0.381) (layer B.Cu) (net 6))
 (segment (start 157.2775 186.075) (end 157.2775 185.77901) (width 0.381) (layer F.Cu) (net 6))
 (segment (start 153.6446 181.8894) (end 153.3206 181.8894) (width 0.254) (layer B.Cu) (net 6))
 (segment (start 158.175 176.425) (end 154.120787 176.425) (width 0.381) (layer F.Cu) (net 7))
 (segment (start 154.120787 176.425) (end 153.3206 177.225187) (width 0.381) (layer F.Cu) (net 7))
 (segment (start 153.3206 177.225187) (end 153.3206 178.6394) (width 0.381) (layer F.Cu) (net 7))
 (segment (start 166.175 178.0975) (end 166.175 177.225) (width 0.381) (layer F.Cu) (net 7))
 (segment (start 157.7025 176.8975) (end 157.7025 177.7) (width 0.381) (layer F.Cu) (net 7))
 (segment (start 158.175 176.425) (end 157.7025 176.8975) (width 0.381) (layer F.Cu) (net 7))
 (segment (start 165.375 176.425) (end 158.175 176.425) (width 0.381) (layer F.Cu) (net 7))
 (segment (start 166.175 177.225) (end 165.375 176.425) (width 0.381) (layer F.Cu) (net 7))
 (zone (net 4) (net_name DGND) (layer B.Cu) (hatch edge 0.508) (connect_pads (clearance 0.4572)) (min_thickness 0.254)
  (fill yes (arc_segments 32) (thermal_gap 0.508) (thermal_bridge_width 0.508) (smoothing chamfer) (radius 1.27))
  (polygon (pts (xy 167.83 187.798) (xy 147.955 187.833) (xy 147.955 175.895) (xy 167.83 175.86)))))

